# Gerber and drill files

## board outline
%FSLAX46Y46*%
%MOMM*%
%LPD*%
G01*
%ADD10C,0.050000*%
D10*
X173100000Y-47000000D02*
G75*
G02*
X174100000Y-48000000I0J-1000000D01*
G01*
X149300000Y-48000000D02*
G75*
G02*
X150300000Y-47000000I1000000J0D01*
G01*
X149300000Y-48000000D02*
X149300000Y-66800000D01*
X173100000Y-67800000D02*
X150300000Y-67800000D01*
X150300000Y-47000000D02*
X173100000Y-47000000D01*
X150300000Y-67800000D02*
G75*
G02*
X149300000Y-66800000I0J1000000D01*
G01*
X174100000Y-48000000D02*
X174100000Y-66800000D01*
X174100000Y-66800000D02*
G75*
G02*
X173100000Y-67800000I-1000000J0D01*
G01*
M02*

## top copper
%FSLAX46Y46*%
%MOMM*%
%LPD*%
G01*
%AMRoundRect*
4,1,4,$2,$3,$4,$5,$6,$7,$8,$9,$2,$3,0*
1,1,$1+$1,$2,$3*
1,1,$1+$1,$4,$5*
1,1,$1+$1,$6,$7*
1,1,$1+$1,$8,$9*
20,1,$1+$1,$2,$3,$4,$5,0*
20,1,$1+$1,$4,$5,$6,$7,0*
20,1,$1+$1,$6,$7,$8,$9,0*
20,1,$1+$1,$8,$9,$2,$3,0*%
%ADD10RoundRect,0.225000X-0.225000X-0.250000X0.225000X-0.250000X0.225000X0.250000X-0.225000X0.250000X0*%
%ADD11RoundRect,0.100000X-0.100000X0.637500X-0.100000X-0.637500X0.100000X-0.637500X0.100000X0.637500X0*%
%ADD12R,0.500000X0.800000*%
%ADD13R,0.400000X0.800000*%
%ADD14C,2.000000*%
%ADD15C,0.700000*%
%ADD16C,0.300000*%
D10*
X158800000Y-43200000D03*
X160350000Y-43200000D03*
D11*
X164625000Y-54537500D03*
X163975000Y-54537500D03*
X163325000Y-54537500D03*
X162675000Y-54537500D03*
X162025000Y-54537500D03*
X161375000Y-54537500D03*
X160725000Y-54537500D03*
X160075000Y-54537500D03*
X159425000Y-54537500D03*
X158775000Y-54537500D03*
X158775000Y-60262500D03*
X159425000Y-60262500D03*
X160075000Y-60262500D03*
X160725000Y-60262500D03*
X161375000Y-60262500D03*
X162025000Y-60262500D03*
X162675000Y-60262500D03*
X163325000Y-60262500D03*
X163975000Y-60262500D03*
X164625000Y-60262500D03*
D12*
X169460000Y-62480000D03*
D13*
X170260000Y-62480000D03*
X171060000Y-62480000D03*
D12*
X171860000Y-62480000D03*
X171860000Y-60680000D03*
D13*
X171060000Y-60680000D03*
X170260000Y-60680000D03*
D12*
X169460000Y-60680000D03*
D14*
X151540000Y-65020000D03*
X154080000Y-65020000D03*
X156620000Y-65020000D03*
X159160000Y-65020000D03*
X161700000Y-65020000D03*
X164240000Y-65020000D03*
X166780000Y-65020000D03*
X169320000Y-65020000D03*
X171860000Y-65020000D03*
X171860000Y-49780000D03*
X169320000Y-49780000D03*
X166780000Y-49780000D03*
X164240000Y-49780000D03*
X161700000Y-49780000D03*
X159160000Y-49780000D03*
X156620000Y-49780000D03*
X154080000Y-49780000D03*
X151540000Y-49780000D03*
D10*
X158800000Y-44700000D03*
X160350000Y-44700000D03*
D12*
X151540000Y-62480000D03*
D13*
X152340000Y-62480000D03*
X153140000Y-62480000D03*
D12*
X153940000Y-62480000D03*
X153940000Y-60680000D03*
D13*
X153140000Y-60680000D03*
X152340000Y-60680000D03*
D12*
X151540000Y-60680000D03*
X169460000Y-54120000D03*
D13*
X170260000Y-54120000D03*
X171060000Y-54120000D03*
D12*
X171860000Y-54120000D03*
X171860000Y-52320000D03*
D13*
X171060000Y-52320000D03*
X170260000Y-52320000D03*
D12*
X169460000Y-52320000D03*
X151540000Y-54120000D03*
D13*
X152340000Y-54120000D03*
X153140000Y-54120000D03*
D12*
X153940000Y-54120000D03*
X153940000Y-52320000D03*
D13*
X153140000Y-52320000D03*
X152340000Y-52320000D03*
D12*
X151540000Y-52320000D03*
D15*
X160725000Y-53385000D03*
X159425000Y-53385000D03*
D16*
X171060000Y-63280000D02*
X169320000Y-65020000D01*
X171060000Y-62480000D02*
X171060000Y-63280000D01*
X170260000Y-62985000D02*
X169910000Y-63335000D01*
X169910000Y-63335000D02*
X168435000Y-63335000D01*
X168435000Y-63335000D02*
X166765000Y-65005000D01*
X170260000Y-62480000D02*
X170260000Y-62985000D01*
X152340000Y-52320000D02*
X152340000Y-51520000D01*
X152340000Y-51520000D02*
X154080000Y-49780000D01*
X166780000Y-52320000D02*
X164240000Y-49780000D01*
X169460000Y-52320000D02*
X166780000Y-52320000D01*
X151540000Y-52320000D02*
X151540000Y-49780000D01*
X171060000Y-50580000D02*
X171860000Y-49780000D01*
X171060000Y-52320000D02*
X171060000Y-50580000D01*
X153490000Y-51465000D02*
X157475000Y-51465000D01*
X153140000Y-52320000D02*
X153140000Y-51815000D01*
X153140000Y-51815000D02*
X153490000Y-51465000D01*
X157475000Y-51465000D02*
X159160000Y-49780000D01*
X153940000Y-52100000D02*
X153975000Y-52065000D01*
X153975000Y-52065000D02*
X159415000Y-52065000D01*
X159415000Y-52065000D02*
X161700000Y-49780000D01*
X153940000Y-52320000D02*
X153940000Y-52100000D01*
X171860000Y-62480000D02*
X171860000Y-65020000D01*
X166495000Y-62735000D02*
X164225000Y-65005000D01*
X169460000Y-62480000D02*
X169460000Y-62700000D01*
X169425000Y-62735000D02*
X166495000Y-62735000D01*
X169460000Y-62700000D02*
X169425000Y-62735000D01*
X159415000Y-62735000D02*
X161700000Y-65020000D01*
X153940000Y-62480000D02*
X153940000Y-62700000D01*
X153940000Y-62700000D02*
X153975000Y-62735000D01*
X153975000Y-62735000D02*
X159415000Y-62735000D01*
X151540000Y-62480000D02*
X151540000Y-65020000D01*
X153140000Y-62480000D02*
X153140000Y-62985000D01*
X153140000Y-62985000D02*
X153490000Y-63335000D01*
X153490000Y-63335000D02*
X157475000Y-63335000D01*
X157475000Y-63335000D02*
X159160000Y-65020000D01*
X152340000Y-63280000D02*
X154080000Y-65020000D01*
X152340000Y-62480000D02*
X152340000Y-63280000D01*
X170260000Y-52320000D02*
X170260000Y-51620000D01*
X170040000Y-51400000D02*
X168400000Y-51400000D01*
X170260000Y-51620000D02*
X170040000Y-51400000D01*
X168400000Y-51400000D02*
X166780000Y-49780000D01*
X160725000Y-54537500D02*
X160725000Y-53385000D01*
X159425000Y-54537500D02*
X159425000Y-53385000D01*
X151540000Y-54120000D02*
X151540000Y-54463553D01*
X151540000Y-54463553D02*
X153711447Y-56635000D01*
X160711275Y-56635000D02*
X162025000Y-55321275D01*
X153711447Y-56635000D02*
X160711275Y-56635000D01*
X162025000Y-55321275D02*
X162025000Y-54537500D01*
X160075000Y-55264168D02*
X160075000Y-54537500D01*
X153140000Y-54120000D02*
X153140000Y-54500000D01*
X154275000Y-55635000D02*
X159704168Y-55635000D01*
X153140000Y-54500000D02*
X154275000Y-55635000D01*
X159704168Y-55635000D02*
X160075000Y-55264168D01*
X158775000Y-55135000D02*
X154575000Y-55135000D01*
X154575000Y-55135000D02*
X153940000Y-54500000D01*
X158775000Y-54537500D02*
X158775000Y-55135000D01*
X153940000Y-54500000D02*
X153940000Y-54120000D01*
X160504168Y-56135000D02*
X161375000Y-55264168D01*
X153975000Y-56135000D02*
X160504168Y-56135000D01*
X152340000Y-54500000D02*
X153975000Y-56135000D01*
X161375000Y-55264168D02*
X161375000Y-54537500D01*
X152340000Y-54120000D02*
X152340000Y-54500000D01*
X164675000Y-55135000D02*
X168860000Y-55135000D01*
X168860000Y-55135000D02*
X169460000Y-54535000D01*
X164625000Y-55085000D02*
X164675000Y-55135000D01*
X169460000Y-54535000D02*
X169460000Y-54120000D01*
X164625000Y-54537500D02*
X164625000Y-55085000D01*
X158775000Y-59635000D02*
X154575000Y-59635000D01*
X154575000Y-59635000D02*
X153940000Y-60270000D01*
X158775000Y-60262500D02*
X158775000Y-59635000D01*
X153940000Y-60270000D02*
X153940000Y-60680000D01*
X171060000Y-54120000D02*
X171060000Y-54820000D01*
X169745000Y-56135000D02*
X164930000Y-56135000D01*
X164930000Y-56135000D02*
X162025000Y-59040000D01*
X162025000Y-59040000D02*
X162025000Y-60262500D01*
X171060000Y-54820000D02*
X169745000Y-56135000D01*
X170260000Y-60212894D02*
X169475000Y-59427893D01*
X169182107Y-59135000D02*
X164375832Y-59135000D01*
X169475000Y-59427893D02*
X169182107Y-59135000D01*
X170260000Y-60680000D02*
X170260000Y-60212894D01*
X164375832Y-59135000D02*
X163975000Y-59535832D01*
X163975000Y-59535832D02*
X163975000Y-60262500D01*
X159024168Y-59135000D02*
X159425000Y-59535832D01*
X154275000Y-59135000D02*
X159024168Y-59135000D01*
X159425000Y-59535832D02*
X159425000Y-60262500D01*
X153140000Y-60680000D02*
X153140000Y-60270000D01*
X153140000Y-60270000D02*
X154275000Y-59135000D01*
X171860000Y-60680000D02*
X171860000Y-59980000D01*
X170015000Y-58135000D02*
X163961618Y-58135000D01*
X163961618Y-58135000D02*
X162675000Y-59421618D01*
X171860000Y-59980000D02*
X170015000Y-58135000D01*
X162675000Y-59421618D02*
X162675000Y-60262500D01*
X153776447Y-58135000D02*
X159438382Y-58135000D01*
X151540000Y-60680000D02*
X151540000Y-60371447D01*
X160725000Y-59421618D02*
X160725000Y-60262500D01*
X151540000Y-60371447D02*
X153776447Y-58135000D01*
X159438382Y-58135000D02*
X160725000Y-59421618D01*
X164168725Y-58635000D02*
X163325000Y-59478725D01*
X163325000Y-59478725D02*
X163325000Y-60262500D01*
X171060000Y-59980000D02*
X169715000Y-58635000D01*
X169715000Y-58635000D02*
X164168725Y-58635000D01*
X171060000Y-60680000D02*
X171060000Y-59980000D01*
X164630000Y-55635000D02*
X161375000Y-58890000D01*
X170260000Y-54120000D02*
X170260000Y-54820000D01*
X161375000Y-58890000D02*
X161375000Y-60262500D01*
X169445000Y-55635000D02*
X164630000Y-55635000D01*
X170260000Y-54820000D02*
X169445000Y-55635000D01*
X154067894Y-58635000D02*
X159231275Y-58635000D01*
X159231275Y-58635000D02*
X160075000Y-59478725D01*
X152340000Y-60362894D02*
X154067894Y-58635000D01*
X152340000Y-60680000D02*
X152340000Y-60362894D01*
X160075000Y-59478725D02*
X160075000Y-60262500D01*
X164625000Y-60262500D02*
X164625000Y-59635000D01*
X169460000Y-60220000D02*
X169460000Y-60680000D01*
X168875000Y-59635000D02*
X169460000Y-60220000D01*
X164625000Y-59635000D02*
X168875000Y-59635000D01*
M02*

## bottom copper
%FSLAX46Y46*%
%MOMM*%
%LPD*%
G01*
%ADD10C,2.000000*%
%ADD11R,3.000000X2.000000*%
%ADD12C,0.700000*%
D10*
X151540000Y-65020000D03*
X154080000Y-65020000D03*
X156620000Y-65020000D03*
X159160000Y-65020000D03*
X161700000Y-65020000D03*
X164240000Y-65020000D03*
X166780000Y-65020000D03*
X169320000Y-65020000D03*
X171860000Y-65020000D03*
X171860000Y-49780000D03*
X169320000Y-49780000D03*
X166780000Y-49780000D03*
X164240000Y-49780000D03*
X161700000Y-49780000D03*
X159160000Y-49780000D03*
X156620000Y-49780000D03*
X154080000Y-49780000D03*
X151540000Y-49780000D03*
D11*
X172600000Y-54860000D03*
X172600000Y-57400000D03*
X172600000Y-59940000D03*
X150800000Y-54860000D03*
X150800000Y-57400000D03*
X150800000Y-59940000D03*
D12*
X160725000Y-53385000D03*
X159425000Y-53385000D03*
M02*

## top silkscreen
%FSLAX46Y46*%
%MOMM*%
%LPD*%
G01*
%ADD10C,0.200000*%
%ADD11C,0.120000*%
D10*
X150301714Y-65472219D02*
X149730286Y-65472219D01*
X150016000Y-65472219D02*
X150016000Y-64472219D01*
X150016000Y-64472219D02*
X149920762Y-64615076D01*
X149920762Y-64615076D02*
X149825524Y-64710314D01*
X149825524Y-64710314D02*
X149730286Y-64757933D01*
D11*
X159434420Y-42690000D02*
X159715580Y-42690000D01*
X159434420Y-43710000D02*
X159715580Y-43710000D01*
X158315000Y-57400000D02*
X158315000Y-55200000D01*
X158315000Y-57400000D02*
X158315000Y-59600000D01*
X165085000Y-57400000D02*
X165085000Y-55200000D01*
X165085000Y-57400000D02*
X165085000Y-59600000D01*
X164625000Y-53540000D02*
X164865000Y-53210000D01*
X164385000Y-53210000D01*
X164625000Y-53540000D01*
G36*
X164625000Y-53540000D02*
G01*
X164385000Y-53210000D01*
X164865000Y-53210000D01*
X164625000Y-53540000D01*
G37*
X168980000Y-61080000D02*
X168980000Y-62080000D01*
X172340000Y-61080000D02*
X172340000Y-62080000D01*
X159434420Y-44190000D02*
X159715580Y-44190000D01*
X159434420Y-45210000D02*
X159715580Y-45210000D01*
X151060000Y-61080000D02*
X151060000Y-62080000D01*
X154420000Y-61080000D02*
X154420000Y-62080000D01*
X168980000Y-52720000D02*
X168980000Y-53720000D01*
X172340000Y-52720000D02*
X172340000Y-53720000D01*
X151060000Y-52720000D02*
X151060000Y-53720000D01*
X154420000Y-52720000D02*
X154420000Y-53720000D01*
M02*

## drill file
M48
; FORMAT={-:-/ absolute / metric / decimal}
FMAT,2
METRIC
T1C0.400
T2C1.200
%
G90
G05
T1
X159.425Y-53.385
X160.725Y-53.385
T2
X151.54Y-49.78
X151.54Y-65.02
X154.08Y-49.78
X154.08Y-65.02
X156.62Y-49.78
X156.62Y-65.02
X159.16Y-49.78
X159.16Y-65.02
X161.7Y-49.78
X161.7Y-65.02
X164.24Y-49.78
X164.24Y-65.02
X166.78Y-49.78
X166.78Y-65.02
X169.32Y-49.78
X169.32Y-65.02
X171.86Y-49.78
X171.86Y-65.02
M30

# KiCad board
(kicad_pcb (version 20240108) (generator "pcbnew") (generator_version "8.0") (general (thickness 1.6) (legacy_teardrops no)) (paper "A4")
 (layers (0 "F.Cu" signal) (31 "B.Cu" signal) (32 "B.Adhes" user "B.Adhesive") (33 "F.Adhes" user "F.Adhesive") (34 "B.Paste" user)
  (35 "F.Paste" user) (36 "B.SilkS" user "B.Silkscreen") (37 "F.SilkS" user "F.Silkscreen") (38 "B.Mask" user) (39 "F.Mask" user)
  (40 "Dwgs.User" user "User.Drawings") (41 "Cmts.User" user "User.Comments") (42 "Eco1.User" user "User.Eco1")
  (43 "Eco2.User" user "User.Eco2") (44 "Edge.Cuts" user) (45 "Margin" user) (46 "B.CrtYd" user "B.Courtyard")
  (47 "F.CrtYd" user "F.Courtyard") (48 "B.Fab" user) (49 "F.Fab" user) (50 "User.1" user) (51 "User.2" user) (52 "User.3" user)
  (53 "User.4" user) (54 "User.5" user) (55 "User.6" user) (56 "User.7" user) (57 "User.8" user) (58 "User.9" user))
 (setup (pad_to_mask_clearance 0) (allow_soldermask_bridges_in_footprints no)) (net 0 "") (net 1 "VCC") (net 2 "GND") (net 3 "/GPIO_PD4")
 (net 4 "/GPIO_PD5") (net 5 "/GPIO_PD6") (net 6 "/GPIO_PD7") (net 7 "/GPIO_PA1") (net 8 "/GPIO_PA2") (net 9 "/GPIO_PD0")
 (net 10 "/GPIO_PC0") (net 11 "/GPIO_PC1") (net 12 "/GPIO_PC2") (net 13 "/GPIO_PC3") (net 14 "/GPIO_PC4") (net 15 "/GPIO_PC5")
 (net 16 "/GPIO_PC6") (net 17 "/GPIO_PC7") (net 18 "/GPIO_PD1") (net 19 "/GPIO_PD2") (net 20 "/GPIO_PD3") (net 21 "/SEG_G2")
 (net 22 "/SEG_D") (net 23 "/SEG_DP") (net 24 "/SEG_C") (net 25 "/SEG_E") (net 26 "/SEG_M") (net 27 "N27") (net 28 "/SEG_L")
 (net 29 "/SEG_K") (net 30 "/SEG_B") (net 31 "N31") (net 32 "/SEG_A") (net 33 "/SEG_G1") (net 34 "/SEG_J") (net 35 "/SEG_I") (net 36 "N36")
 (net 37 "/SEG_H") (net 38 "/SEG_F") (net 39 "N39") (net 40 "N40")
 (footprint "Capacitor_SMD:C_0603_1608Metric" (layer "F.Cu") (at 159.575 43.2)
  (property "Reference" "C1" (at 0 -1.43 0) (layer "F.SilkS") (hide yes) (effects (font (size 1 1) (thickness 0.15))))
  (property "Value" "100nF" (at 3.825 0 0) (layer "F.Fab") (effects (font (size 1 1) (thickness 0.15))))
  (fp_line (start -0.14058 -0.51) (end 0.14058 -0.51) (stroke (width 0.12) (type solid)) (layer "F.SilkS"))
  (fp_line (start -0.14058 0.51) (end 0.14058 0.51) (stroke (width 0.12) (type solid)) (layer "F.SilkS"))
  (pad "1" smd roundrect (at -0.775 0) (size 0.9 0.95) (layers "F.Cu" "F.Paste" "F.Mask") (roundrect_rratio 0.25) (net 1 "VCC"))
  (pad "2" smd roundrect (at 0.775 0) (size 0.9 0.95) (layers "F.Cu" "F.Paste" "F.Mask") (roundrect_rratio 0.25) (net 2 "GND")))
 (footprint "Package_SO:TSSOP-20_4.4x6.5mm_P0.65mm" (layer "F.Cu") (at 161.7 57.4 -90)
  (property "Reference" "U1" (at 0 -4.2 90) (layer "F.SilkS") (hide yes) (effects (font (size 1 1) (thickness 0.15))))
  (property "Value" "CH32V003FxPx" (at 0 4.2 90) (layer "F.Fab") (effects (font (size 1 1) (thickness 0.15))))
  (fp_line (start 0 3.385) (end -2.2 3.385) (stroke (width 0.12) (type solid)) (layer "F.SilkS"))
  (fp_line (start 0 3.385) (end 2.2 3.385) (stroke (width 0.12) (type solid)) (layer "F.SilkS"))
  (fp_line (start 0 -3.385) (end -2.2 -3.385) (stroke (width 0.12) (type solid)) (layer "F.SilkS"))
  (fp_line (start 0 -3.385) (end 2.2 -3.385) (stroke (width 0.12) (type solid)) (layer "F.SilkS"))
  (fp_poly
   (pts (xy -3.86 -2.925) (xy -4.19 -3.165) (xy -4.19 -2.685) (xy -3.86 -2.925)) (stroke (width 0.12) (type solid)) (fill solid)
   (layer "F.SilkS"))
  (pad "1" smd roundrect (at -2.8625 -2.925 270) (size 1.475 0.4) (layers "F.Cu" "F.Paste" "F.Mask") (roundrect_rratio 0.25)
   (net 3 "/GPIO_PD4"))
  (pad "2" smd roundrect (at -2.8625 -2.275 270) (size 1.475 0.4) (layers "F.Cu" "F.Paste" "F.Mask") (roundrect_rratio 0.25)
   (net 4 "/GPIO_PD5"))
  (pad "3" smd roundrect (at -2.8625 -1.625 270) (size 1.475 0.4) (layers "F.Cu" "F.Paste" "F.Mask") (roundrect_rratio 0.25)
   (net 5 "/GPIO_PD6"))
  (pad "4" smd roundrect (at -2.8625 -0.975 270) (size 1.475 0.4) (layers "F.Cu" "F.Paste" "F.Mask") (roundrect_rratio 0.25)
   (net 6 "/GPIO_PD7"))
  (pad "5" smd roundrect (at -2.8625 -0.325 270) (size 1.475 0.4) (layers "F.Cu" "F.Paste" "F.Mask") (roundrect_rratio 0.25)
   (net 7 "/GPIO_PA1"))
  (pad "6" smd roundrect (at -2.8625 0.325 270) (size 1.475 0.4) (layers "F.Cu" "F.Paste" "F.Mask") (roundrect_rratio 0.25)
   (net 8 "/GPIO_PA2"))
  (pad "7" smd roundrect (at -2.8625 0.975 270) (size 1.475 0.4) (layers "F.Cu" "F.Paste" "F.Mask") (roundrect_rratio 0.25) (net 2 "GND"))
  (pad "8" smd roundrect (at -2.8625 1.625 270) (size 1.475 0.4) (layers "F.Cu" "F.Paste" "F.Mask") (roundrect_rratio 0.25)
   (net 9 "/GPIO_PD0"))
  (pad "9" smd roundrect (at -2.8625 2.275 270) (size 1.475 0.4) (layers "F.Cu" "F.Paste" "F.Mask") (roundrect_rratio 0.25) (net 1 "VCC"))
  (pad "10" smd roundrect (at -2.8625 2.925 270) (size 1.475 0.4) (layers "F.Cu" "F.Paste" "F.Mask") (roundrect_rratio 0.25)
   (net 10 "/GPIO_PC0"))
  (pad "11" smd roundrect (at 2.8625 2.925 270) (size 1.475 0.4) (layers "F.Cu" "F.Paste" "F.Mask") (roundrect_rratio 0.25)
   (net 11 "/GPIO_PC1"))
  (pad "12" smd roundrect (at 2.8625 2.275 270) (size 1.475 0.4) (layers "F.Cu" "F.Paste" "F.Mask") (roundrect_rratio 0.25)
   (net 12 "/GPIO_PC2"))
  (pad "13" smd roundrect (at 2.8625 1.625 270) (size 1.475 0.4) (layers "F.Cu" "F.Paste" "F.Mask") (roundrect_rratio 0.25)
   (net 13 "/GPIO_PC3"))
  (pad "14" smd roundrect (at 2.8625 0.975 270) (size 1.475 0.4) (layers "F.Cu" "F.Paste" "F.Mask") (roundrect_rratio 0.25)
   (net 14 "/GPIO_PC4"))
  (pad "15" smd roundrect (at 2.8625 0.325 270) (size 1.475 0.4) (layers "F.Cu" "F.Paste" "F.Mask") (roundrect_rratio 0.25)
   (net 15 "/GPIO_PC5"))
  (pad "16" smd roundrect (at 2.8625 -0.325 270) (size 1.475 0.4) (layers "F.Cu" "F.Paste" "F.Mask") (roundrect_rratio 0.25)
   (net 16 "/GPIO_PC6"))
  (pad "17" smd roundrect (at 2.8625 -0.975 270) (size 1.475 0.4) (layers "F.Cu" "F.Paste" "F.Mask") (roundrect_rratio 0.25)
   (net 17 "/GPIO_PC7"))
  (pad "18" smd roundrect (at 2.8625 -1.625 270) (size 1.475 0.4) (layers "F.Cu" "F.Paste" "F.Mask") (roundrect_rratio 0.25)
   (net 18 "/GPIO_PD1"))
  (pad "19" smd roundrect (at 2.8625 -2.275 270) (size 1.475 0.4) (layers "F.Cu" "F.Paste" "F.Mask") (roundrect_rratio 0.25)
   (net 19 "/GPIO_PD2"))
  (pad "20" smd roundrect (at 2.8625 -2.925 270) (size 1.475 0.4) (layers "F.Cu" "F.Paste" "F.Mask") (roundrect_rratio 0.25)
   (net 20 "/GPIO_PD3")))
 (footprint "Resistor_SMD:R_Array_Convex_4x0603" (layer "F.Cu") (at 170.66 61.58 90)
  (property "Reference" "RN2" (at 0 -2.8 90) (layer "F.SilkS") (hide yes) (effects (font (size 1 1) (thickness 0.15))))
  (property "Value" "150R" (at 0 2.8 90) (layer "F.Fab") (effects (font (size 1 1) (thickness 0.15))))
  (fp_line (start 0.5 -1.68) (end -0.5 -1.68) (stroke (width 0.12) (type solid)) (layer "F.SilkS"))
  (fp_line (start 0.5 1.68) (end -0.5 1.68) (stroke (width 0.12) (type solid)) (layer "F.SilkS"))
  (pad "1" smd rect (at -0.9 -1.2 90) (size 0.8 0.5) (layers "F.Cu" "F.Paste" "F.Mask") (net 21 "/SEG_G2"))
  (pad "2" smd rect (at -0.9 -0.4 90) (size 0.8 0.4) (layers "F.Cu" "F.Paste" "F.Mask") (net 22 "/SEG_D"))
  (pad "3" smd rect (at -0.9 0.4 90) (size 0.8 0.4) (layers "F.Cu" "F.Paste" "F.Mask") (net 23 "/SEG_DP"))
  (pad "4" smd rect (at -0.9 1.2 90) (size 0.8 0.5) (layers "F.Cu" "F.Paste" "F.Mask") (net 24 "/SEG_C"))
  (pad "5" smd rect (at 0.9 1.2 90) (size 0.8 0.5) (layers "F.Cu" "F.Paste" "F.Mask") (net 17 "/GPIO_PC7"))
  (pad "6" smd rect (at 0.9 0.4 90) (size 0.8 0.4) (layers "F.Cu" "F.Paste" "F.Mask") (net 18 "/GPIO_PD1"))
  (pad "7" smd rect (at 0.9 -0.4 90) (size 0.8 0.4) (layers "F.Cu" "F.Paste" "F.Mask") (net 19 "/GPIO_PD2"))
  (pad "8" smd rect (at 0.9 -1.2 90) (size 0.8 0.5) (layers "F.Cu" "F.Paste" "F.Mask") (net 20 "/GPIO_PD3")))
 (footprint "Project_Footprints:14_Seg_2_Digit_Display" (layer "F.Cu") (at 161.7 57.4)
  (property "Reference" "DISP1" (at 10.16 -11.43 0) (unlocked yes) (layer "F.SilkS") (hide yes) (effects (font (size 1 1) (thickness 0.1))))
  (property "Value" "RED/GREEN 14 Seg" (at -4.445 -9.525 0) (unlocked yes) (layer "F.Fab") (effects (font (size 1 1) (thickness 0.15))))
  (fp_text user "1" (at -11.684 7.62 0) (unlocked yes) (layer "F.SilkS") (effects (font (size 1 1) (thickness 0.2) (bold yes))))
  (pad "1" thru_hole circle (at -10.16 7.62) (size 2 2) (drill 1.2) (layers "*.Cu" "*.Mask") (remove_unused_layers no) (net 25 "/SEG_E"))
  (pad "2" thru_hole circle (at -7.62 7.62) (size 2 2) (drill 1.2) (layers "*.Cu" "*.Mask") (remove_unused_layers no) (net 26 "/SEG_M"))
  (pad "3" thru_hole circle (at -5.08 7.62) (size 2 2) (drill 1.2) (layers "*.Cu" "*.Mask") (remove_unused_layers no) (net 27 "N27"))
  (pad "4" thru_hole circle (at -2.54 7.62) (size 2 2) (drill 1.2) (layers "*.Cu" "*.Mask") (remove_unused_layers no) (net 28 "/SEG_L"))
  (pad "5" thru_hole circle (at 0 7.62) (size 2 2) (drill 1.2) (layers "*.Cu" "*.Mask") (remove_unused_layers no) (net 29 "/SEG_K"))
  (pad "6" thru_hole circle (at 2.54 7.62) (size 2 2) (drill 1.2) (layers "*.Cu" "*.Mask") (remove_unused_layers no) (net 21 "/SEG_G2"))
  (pad "7" thru_hole circle (at 5.08 7.62) (size 2 2) (drill 1.2) (layers "*.Cu" "*.Mask") (remove_unused_layers no) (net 22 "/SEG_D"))
  (pad "8" thru_hole circle (at 7.62 7.62) (size 2 2) (drill 1.2) (layers "*.Cu" "*.Mask") (remove_unused_layers no) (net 23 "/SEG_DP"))
  (pad "9" thru_hole circle (at 10.16 7.62) (size 2 2) (drill 1.2) (layers "*.Cu" "*.Mask") (remove_unused_layers no) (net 24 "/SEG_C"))
  (pad "10" thru_hole circle (at 10.16 -7.62) (size 2 2) (drill 1.2) (layers "*.Cu" "*.Mask") (remove_unused_layers no) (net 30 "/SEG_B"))
  (pad "11" thru_hole circle (at 7.62 -7.62) (size 2 2) (drill 1.2) (layers "*.Cu" "*.Mask") (remove_unused_layers no) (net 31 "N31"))
  (pad "12" thru_hole circle (at 5.08 -7.62) (size 2 2) (drill 1.2) (layers "*.Cu" "*.Mask") (remove_unused_layers no) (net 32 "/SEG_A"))
  (pad "13" thru_hole circle (at 2.54 -7.62) (size 2 2) (drill 1.2) (layers "*.Cu" "*.Mask") (remove_unused_layers no) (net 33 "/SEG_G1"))
  (pad "14" thru_hole circle (at 0 -7.62) (size 2 2) (drill 1.2) (layers "*.Cu" "*.Mask") (remove_unused_layers no) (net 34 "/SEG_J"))
  (pad "15" thru_hole circle (at -2.54 -7.62) (size 2 2) (drill 1.2) (layers "*.Cu" "*.Mask") (remove_unused_layers no) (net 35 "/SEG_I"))
  (pad "16" thru_hole circle (at -5.08 -7.62) (size 2 2) (drill 1.2) (layers "*.Cu" "*.Mask") (remove_unused_layers no) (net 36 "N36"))
  (pad "17" thru_hole circle (at -7.62 -7.62) (size 2 2) (drill 1.2) (layers "*.Cu" "*.Mask") (remove_unused_layers no) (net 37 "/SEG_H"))
  (pad "18" thru_hole circle (at -10.16 -7.62) (size 2 2) (drill 1.2) (layers "*.Cu" "*.Mask") (remove_unused_layers no) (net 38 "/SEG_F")))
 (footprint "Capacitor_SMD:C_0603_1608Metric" (layer "F.Cu") (at 159.575 44.7)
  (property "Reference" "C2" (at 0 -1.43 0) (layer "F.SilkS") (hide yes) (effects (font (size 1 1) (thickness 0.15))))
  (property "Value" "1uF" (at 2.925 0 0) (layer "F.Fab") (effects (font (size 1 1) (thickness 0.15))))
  (fp_line (start -0.14058 -0.51) (end 0.14058 -0.51) (stroke (width 0.12) (type solid)) (layer "F.SilkS"))
  (fp_line (start -0.14058 0.51) (end 0.14058 0.51) (stroke (width 0.12) (type solid)) (layer "F.SilkS"))
  (pad "1" smd roundrect (at -0.775 0) (size 0.9 0.95) (layers "F.Cu" "F.Paste" "F.Mask") (roundrect_rratio 0.25) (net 1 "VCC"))
  (pad "2" smd roundrect (at 0.775 0) (size 0.9 0.95) (layers "F.Cu" "F.Paste" "F.Mask") (roundrect_rratio 0.25) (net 2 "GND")))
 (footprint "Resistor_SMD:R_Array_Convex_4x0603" (layer "F.Cu") (at 152.74 61.58 90)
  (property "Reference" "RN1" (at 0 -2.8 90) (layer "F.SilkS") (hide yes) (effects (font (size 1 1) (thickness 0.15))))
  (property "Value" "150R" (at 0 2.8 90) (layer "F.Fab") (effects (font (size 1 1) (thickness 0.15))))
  (fp_line (start 0.5 -1.68) (end -0.5 -1.68) (stroke (width 0.12) (type solid)) (layer "F.SilkS"))
  (fp_line (start 0.5 1.68) (end -0.5 1.68) (stroke (width 0.12) (type solid)) (layer "F.SilkS"))
  (pad "1" smd rect (at -0.9 -1.2 90) (size 0.8 0.5) (layers "F.Cu" "F.Paste" "F.Mask") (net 25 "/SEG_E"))
  (pad "2" smd rect (at -0.9 -0.4 90) (size 0.8 0.4) (layers "F.Cu" "F.Paste" "F.Mask") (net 26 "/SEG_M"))
  (pad "3" smd rect (at -0.9 0.4 90) (size 0.8 0.4) (layers "F.Cu" "F.Paste" "F.Mask") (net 28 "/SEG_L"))
  (pad "4" smd rect (at -0.9 1.2 90) (size 0.8 0.5) (layers "F.Cu" "F.Paste" "F.Mask") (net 29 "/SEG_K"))
  (pad "5" smd rect (at 0.9 1.2 90) (size 0.8 0.5) (layers "F.Cu" "F.Paste" "F.Mask") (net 11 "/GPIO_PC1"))
  (pad "6" smd rect (at 0.9 0.4 90) (size 0.8 0.4) (layers "F.Cu" "F.Paste" "F.Mask") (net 12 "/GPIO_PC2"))
  (pad "7" smd rect (at 0.9 -0.4 90) (size 0.8 0.4) (layers "F.Cu" "F.Paste" "F.Mask") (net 13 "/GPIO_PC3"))
  (pad "8" smd rect (at 0.9 -1.2 90) (size 0.8 0.5) (layers "F.Cu" "F.Paste" "F.Mask") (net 14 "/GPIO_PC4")))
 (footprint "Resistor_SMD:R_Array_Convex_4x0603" (layer "F.Cu") (at 170.66 53.22 90)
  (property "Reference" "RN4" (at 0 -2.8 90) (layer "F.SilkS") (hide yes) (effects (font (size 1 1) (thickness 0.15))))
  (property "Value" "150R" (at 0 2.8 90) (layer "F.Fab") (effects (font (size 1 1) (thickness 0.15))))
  (fp_line (start 0.5 -1.68) (end -0.5 -1.68) (stroke (width 0.12) (type solid)) (layer "F.SilkS"))
  (fp_line (start 0.5 1.68) (end -0.5 1.68) (stroke (width 0.12) (type solid)) (layer "F.SilkS"))
  (pad "1" smd rect (at -0.9 -1.2 90) (size 0.8 0.5) (layers "F.Cu" "F.Paste" "F.Mask") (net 3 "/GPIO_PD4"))
  (pad "2" smd rect (at -0.9 -0.4 90) (size 0.8 0.4) (layers "F.Cu" "F.Paste" "F.Mask") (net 15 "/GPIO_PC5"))
  (pad "3" smd rect (at -0.9 0.4 90) (size 0.8 0.4) (layers "F.Cu" "F.Paste" "F.Mask") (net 16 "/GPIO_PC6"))
  (pad "4" smd rect (at -0.9 1.2 90) (size 0.8 0.5) (layers "F.Cu" "F.Paste" "F.Mask") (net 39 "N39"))
  (pad "5" smd rect (at 0.9 1.2 90) (size 0.8 0.5) (layers "F.Cu" "F.Paste" "F.Mask") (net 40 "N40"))
  (pad "6" smd rect (at 0.9 0.4 90) (size 0.8 0.4) (layers "F.Cu" "F.Paste" "F.Mask") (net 30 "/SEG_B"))
  (pad "7" smd rect (at 0.9 -0.4 90) (size 0.8 0.4) (layers "F.Cu" "F.Paste" "F.Mask") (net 32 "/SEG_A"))
  (pad "8" smd rect (at 0.9 -1.2 90) (size 0.8 0.5) (layers "F.Cu" "F.Paste" "F.Mask") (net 33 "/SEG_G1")))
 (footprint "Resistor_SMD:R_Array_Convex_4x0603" (layer "F.Cu") (at 152.74 53.22 90)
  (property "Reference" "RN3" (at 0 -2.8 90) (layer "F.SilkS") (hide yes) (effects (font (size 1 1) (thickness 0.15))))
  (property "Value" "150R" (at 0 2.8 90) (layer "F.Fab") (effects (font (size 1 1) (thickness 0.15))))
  (fp_line (start 0.5 -1.68) (end -0.5 -1.68) (stroke (width 0.12) (type solid)) (layer "F.SilkS"))
  (fp_line (start 0.5 1.68) (end -0.5 1.68) (stroke (width 0.12) (type solid)) (layer "F.SilkS"))
  (pad "1" smd rect (at -0.9 -1.2 90) (size 0.8 0.5) (layers "F.Cu" "F.Paste" "F.Mask") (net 7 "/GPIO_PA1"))
  (pad "2" smd rect (at -0.9 -0.4 90) (size 0.8 0.4) (layers "F.Cu" "F.Paste" "F.Mask") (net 8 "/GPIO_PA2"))
  (pad "3" smd rect (at -0.9 0.4 90) (size 0.8 0.4) (layers "F.Cu" "F.Paste" "F.Mask") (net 9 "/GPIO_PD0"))
  (pad "4" smd rect (at -0.9 1.2 90) (size 0.8 0.5) (layers "F.Cu" "F.Paste" "F.Mask") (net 10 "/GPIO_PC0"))
  (pad "5" smd rect (at 0.9 1.2 90) (size 0.8 0.5) (layers "F.Cu" "F.Paste" "F.Mask") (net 34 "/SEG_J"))
  (pad "6" smd rect (at 0.9 0.4 90) (size 0.8 0.4) (layers "F.Cu" "F.Paste" "F.Mask") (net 35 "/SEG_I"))
  (pad "7" smd rect (at 0.9 -0.4 90) (size 0.8 0.4) (layers "F.Cu" "F.Paste" "F.Mask") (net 37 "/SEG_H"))
  (pad "8" smd rect (at 0.9 -1.2 90) (size 0.8 0.5) (layers "F.Cu" "F.Paste" "F.Mask") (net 38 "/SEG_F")))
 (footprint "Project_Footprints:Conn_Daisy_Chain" (layer "B.Cu") (at 172.6 57.4 180)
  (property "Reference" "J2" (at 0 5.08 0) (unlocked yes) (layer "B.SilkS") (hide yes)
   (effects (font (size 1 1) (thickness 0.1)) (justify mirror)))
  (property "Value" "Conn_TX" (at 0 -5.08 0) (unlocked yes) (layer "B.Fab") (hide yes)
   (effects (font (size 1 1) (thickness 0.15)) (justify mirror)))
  (pad "1" smd rect (at 0 2.54 180) (size 3 2) (layers "B.Cu" "B.Paste" "B.Mask") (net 1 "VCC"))
  (pad "2" smd rect (at 0 0 180) (size 3 2) (layers "B.Cu" "B.Paste" "B.Mask") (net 4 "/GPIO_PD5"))
  (pad "3" smd rect (at 0 -2.54 180) (size 3 2) (layers "B.Cu" "B.Paste" "B.Mask") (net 2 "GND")))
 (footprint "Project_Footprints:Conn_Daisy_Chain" (layer "B.Cu") (at 150.8 57.4 180)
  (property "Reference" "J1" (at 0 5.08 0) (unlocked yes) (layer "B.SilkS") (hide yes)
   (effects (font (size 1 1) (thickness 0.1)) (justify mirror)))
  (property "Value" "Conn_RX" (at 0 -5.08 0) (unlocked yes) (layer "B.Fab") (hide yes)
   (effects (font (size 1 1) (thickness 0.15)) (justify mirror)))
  (pad "1" smd rect (at 0 2.54 180) (size 3 2) (layers "B.Cu" "B.Paste" "B.Mask") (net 1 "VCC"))
  (pad "2" smd rect (at 0 0 180) (size 3 2) (layers "B.Cu" "B.Paste" "B.Mask") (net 5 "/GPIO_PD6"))
  (pad "3" smd rect (at 0 -2.54 180) (size 3 2) (layers "B.Cu" "B.Paste" "B.Mask") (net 2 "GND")))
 (gr_arc (start 173.1 47) (mid 173.807107 47.292893) (end 174.1 48) (stroke (width 0.05) (type default)) (layer "Edge.Cuts"))
 (gr_arc (start 149.3 48) (mid 149.592893 47.292893) (end 150.3 47) (stroke (width 0.05) (type default)) (layer "Edge.Cuts"))
 (gr_line (start 149.3 48) (end 149.3 66.8) (stroke (width 0.05) (type default)) (layer "Edge.Cuts"))
 (gr_line (start 173.1 67.8) (end 150.3 67.8) (stroke (width 0.05) (type default)) (layer "Edge.Cuts"))
 (gr_line (start 150.3 47) (end 173.1 47) (stroke (width 0.05) (type default)) (layer "Edge.Cuts"))
 (gr_arc (start 150.3 67.8) (mid 149.592893 67.507107) (end 149.3 66.8) (stroke (width 0.05) (type default)) (layer "Edge.Cuts"))
 (gr_line (start 174.1 48) (end 174.1 66.8) (stroke (width 0.05) (type default)) (layer "Edge.Cuts"))
 (gr_arc (start 174.1 66.8) (mid 173.807107 67.507107) (end 173.1 67.8) (stroke (width 0.05) (type default)) (layer "Edge.Cuts"))
 (segment (start 171.06 63.28) (end 169.32 65.02) (width 0.3) (layer "F.Cu") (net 23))
 (segment (start 171.06 62.48) (end 171.06 63.28) (width 0.3) (layer "F.Cu") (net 23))
 (segment (start 170.26 62.985) (end 169.91 63.335) (width 0.3) (layer "F.Cu") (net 22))
 (segment (start 169.91 63.335) (end 168.435 63.335) (width 0.3) (layer "F.Cu") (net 22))
 (segment (start 168.435 63.335) (end 166.765 65.005) (width 0.3) (layer "F.Cu") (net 22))
 (segment (start 170.26 62.48) (end 170.26 62.985) (width 0.3) (layer "F.Cu") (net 22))
 (segment (start 152.34 52.32) (end 152.34 51.52) (width 0.3) (layer "F.Cu") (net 37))
 (segment (start 152.34 51.52) (end 154.08 49.78) (width 0.3) (layer "F.Cu") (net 37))
 (segment (start 166.78 52.32) (end 164.24 49.78) (width 0.3) (layer "F.Cu") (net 33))
 (segment (start 169.46 52.32) (end 166.78 52.32) (width 0.3) (layer "F.Cu") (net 33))
 (segment (start 151.54 52.32) (end 151.54 49.78) (width 0.3) (layer "F.Cu") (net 38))
 (segment (start 171.06 50.58) (end 171.86 49.78) (width 0.3) (layer "F.Cu") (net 30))
 (segment (start 171.06 52.32) (end 171.06 50.58) (width 0.3) (layer "F.Cu") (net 30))
 (segment (start 153.49 51.465) (end 157.475 51.465) (width 0.3) (layer "F.Cu") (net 35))
 (segment (start 153.14 52.32) (end 153.14 51.815) (width 0.3) (layer "F.Cu") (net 35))
 (segment (start 153.14 51.815) (end 153.49 51.465) (width 0.3) (layer "F.Cu") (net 35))
 (segment (start 157.475 51.465) (end 159.16 49.78) (width 0.3) (layer "F.Cu") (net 35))
 (segment (start 153.94 52.1) (end 153.975 52.065) (width 0.3) (layer "F.Cu") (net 34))
 (segment (start 153.975 52.065) (end 159.415 52.065) (width 0.3) (layer "F.Cu") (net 34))
 (segment (start 159.415 52.065) (end 161.7 49.78) (width 0.3) (layer "F.Cu") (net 34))
 (segment (start 153.94 52.32) (end 153.94 52.1) (width 0.3) (layer "F.Cu") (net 34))
 (segment (start 171.86 62.48) (end 171.86 65.02) (width 0.3) (layer "F.Cu") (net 24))
 (segment (start 166.495 62.735) (end 164.225 65.005) (width 0.3) (layer "F.Cu") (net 21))
 (segment (start 169.46 62.48) (end 169.46 62.7) (width 0.3) (layer "F.Cu") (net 21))
 (segment (start 169.425 62.735) (end 166.495 62.735) (width 0.3) (layer "F.Cu") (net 21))
 (segment (start 169.46 62.7) (end 169.425 62.735) (width 0.3) (layer "F.Cu") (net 21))
 (segment (start 159.415 62.735) (end 161.7 65.02) (width 0.3) (layer "F.Cu") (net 29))
 (segment (start 153.94 62.48) (end 153.94 62.7) (width 0.3) (layer "F.Cu") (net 29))
 (segment (start 153.94 62.7) (end 153.975 62.735) (width 0.3) (layer "F.Cu") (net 29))
 (segment (start 153.975 62.735) (end 159.415 62.735) (width 0.3) (layer "F.Cu") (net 29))
 (segment (start 151.54 62.48) (end 151.54 65.02) (width 0.3) (layer "F.Cu") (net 25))
 (segment (start 153.14 62.48) (end 153.14 62.985) (width 0.3) (layer "F.Cu") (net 28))
 (segment (start 153.14 62.985) (end 153.49 63.335) (width 0.3) (layer "F.Cu") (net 28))
 (segment (start 153.49 63.335) (end 157.475 63.335) (width 0.3) (layer "F.Cu") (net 28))
 (segment (start 157.475 63.335) (end 159.16 65.02) (width 0.3) (layer "F.Cu") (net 28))
 (segment (start 152.34 63.28) (end 154.08 65.02) (width 0.3) (layer "F.Cu") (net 26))
 (segment (start 152.34 62.48) (end 152.34 63.28) (width 0.3) (layer "F.Cu") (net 26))
 (segment (start 170.26 52.32) (end 170.26 51.62) (width 0.3) (layer "F.Cu") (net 32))
 (segment (start 170.04 51.4) (end 168.4 51.4) (width 0.3) (layer "F.Cu") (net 32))
 (segment (start 170.26 51.62) (end 170.04 51.4) (width 0.3) (layer "F.Cu") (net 32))
 (segment (start 168.4 51.4) (end 166.78 49.78) (width 0.3) (layer "F.Cu") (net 32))
 (segment (start 160.725 54.5375) (end 160.725 53.385) (width 0.3) (layer "F.Cu") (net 2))
 (via (at 160.725 53.385) (size 0.7) (drill 0.4) (layers "F.Cu" "B.Cu") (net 2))
 (segment (start 159.425 54.5375) (end 159.425 53.385) (width 0.3) (layer "F.Cu") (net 1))
 (via (at 159.425 53.385) (size 0.7) (drill 0.4) (layers "F.Cu" "B.Cu") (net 1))
 (segment (start 151.54 54.12) (end 151.54 54.463553) (width 0.3) (layer "F.Cu") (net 7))
 (segment (start 151.54 54.463553) (end 153.711447 56.635) (width 0.3) (layer "F.Cu") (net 7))
 (segment (start 160.711275 56.635) (end 162.025 55.321275) (width 0.3) (layer "F.Cu") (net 7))
 (segment (start 153.711447 56.635) (end 160.711275 56.635) (width 0.3) (layer "F.Cu") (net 7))
 (segment (start 162.025 55.321275) (end 162.025 54.5375) (width 0.3) (layer "F.Cu") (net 7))
 (segment (start 160.075 55.264168) (end 160.075 54.5375) (width 0.3) (layer "F.Cu") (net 9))
 (segment (start 153.14 54.12) (end 153.14 54.5) (width 0.3) (layer "F.Cu") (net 9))
 (segment (start 154.275 55.635) (end 159.704168 55.635) (width 0.3) (layer "F.Cu") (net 9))
 (segment (start 153.14 54.5) (end 154.275 55.635) (width 0.3) (layer "F.Cu") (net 9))
 (segment (start 159.704168 55.635) (end 160.075 55.264168) (width 0.3) (layer "F.Cu") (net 9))
 (segment (start 158.775 55.135) (end 154.575 55.135) (width 0.3) (layer "F.Cu") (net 10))
 (segment (start 154.575 55.135) (end 153.94 54.5) (width 0.3) (layer "F.Cu") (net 10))
 (segment (start 158.775 54.5375) (end 158.775 55.135) (width 0.3) (layer "F.Cu") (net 10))
 (segment (start 153.94 54.5) (end 153.94 54.12) (width 0.3) (layer "F.Cu") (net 10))
 (segment (start 160.504168 56.135) (end 161.375 55.264168) (width 0.3) (layer "F.Cu") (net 8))
 (segment (start 153.975 56.135) (end 160.504168 56.135) (width 0.3) (layer "F.Cu") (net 8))
 (segment (start 152.34 54.5) (end 153.975 56.135) (width 0.3) (layer "F.Cu") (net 8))
 (segment (start 161.375 55.264168) (end 161.375 54.5375) (width 0.3) (layer "F.Cu") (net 8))
 (segment (start 152.34 54.12) (end 152.34 54.5) (width 0.3) (layer "F.Cu") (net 8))
 (segment (start 164.675 55.135) (end 168.86 55.135) (width 0.3) (layer "F.Cu") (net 3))
 (segment (start 168.86 55.135) (end 169.46 54.535) (width 0.3) (layer "F.Cu") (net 3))
 (segment (start 164.625 55.085) (end 164.675 55.135) (width 0.3) (layer "F.Cu") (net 3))
 (segment (start 169.46 54.535) (end 169.46 54.12) (width 0.3) (layer "F.Cu") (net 3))
 (segment (start 164.625 54.5375) (end 164.625 55.085) (width 0.3) (layer "F.Cu") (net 3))
 (segment (start 158.775 59.635) (end 154.575 59.635) (width 0.3) (layer "F.Cu") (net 11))
 (segment (start 154.575 59.635) (end 153.94 60.27) (width 0.3) (layer "F.Cu") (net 11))
 (segment (start 158.775 60.2625) (end 158.775 59.635) (width 0.3) (layer "F.Cu") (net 11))
 (segment (start 153.94 60.27) (end 153.94 60.68) (width 0.3) (layer "F.Cu") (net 11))
 (segment (start 171.06 54.12) (end 171.06 54.82) (width 0.3) (layer "F.Cu") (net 16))
 (segment (start 169.745 56.135) (end 164.93 56.135) (width 0.3) (layer "F.Cu") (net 16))
 (segment (start 164.93 56.135) (end 162.025 59.04) (width 0.3) (layer "F.Cu") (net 16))
 (segment (start 162.025 59.04) (end 162.025 60.2625) (width 0.3) (layer "F.Cu") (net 16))
 (segment (start 171.06 54.82) (end 169.745 56.135) (width 0.3) (layer "F.Cu") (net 16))
 (segment (start 170.26 60.212894) (end 169.475 59.427893) (width 0.3) (layer "F.Cu") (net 19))
 (segment (start 169.182107 59.135) (end 164.375832 59.135) (width 0.3) (layer "F.Cu") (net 19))
 (segment (start 169.475 59.427893) (end 169.182107 59.135) (width 0.3) (layer "F.Cu") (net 19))
 (segment (start 170.26 60.68) (end 170.26 60.212894) (width 0.3) (layer "F.Cu") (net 19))
 (segment (start 164.375832 59.135) (end 163.975 59.535832) (width 0.3) (layer "F.Cu") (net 19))
 (segment (start 163.975 59.535832) (end 163.975 60.2625) (width 0.3) (layer "F.Cu") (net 19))
 (segment (start 159.024168 59.135) (end 159.425 59.535832) (width 0.3) (layer "F.Cu") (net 12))
 (segment (start 154.275 59.135) (end 159.024168 59.135) (width 0.3) (layer "F.Cu") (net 12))
 (segment (start 159.425 59.535832) (end 159.425 60.2625) (width 0.3) (layer "F.Cu") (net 12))
 (segment (start 153.14 60.68) (end 153.14 60.27) (width 0.3) (layer "F.Cu") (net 12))
 (segment (start 153.14 60.27) (end 154.275 59.135) (width 0.3) (layer "F.Cu") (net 12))
 (segment (start 171.86 60.68) (end 171.86 59.98) (width 0.3) (layer "F.Cu") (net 17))
 (segment (start 170.015 58.135) (end 163.961618 58.135) (width 0.3) (layer "F.Cu") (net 17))
 (segment (start 163.961618 58.135) (end 162.675 59.421618) (width 0.3) (layer "F.Cu") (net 17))
 (segment (start 171.86 59.98) (end 170.015 58.135) (width 0.3) (layer "F.Cu") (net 17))
 (segment (start 162.675 59.421618) (end 162.675 60.2625) (width 0.3) (layer "F.Cu") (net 17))
 (segment (start 153.776447 58.135) (end 159.438382 58.135) (width 0.3) (layer "F.Cu") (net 14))
 (segment (start 151.54 60.68) (end 151.54 60.371447) (width 0.3) (layer "F.Cu") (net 14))
 (segment (start 160.725 59.421618) (end 160.725 60.2625) (width 0.3) (layer "F.Cu") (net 14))
 (segment (start 151.54 60.371447) (end 153.776447 58.135) (width 0.3) (layer "F.Cu") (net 14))
 (segment (start 159.438382 58.135) (end 160.725 59.421618) (width 0.3) (layer "F.Cu") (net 14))
 (segment (start 164.168725 58.635) (end 163.325 59.478725) (width 0.3) (layer "F.Cu") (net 18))
 (segment (start 163.325 59.478725) (end 163.325 60.2625) (width 0.3) (layer "F.Cu") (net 18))
 (segment (start 171.06 59.98) (end 169.715 58.635) (width 0.3) (layer "F.Cu") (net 18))
 (segment (start 169.715 58.635) (end 164.168725 58.635) (width 0.3) (layer "F.Cu") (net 18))
 (segment (start 171.06 60.68) (end 171.06 59.98) (width 0.3) (layer "F.Cu") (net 18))
 (segment (start 164.63 55.635) (end 161.375 58.89) (width 0.3) (layer "F.Cu") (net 15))
 (segment (start 170.26 54.12) (end 170.26 54.82) (width 0.3) (layer "F.Cu") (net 15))
 (segment (start 161.375 58.89) (end 161.375 60.2625) (width 0.3) (layer "F.Cu") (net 15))
 (segment (start 169.445 55.635) (end 164.63 55.635) (width 0.3) (layer "F.Cu") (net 15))
 (segment (start 170.26 54.82) (end 169.445 55.635) (width 0.3) (layer "F.Cu") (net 15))
 (segment (start 154.067894 58.635) (end 159.231275 58.635) (width 0.3) (layer "F.Cu") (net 13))
 (segment (start 159.231275 58.635) (end 160.075 59.478725) (width 0.3) (layer "F.Cu") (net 13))
 (segment (start 152.34 60.362894) (end 154.067894 58.635) (width 0.3) (layer "F.Cu") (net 13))
 (segment (start 152.34 60.68) (end 152.34 60.362894) (width 0.3) (layer "F.Cu") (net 13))
 (segment (start 160.075 59.478725) (end 160.075 60.2625) (width 0.3) (layer "F.Cu") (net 13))
 (segment (start 164.625 60.2625) (end 164.625 59.635) (width 0.3) (layer "F.Cu") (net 20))
 (segment (start 169.46 60.22) (end 169.46 60.68) (width 0.3) (layer "F.Cu") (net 20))
 (segment (start 168.875 59.635) (end 169.46 60.22) (width 0.3) (layer "F.Cu") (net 20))
 (segment (start 164.625 59.635) (end 168.875 59.635) (width 0.3) (layer "F.Cu") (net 20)))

